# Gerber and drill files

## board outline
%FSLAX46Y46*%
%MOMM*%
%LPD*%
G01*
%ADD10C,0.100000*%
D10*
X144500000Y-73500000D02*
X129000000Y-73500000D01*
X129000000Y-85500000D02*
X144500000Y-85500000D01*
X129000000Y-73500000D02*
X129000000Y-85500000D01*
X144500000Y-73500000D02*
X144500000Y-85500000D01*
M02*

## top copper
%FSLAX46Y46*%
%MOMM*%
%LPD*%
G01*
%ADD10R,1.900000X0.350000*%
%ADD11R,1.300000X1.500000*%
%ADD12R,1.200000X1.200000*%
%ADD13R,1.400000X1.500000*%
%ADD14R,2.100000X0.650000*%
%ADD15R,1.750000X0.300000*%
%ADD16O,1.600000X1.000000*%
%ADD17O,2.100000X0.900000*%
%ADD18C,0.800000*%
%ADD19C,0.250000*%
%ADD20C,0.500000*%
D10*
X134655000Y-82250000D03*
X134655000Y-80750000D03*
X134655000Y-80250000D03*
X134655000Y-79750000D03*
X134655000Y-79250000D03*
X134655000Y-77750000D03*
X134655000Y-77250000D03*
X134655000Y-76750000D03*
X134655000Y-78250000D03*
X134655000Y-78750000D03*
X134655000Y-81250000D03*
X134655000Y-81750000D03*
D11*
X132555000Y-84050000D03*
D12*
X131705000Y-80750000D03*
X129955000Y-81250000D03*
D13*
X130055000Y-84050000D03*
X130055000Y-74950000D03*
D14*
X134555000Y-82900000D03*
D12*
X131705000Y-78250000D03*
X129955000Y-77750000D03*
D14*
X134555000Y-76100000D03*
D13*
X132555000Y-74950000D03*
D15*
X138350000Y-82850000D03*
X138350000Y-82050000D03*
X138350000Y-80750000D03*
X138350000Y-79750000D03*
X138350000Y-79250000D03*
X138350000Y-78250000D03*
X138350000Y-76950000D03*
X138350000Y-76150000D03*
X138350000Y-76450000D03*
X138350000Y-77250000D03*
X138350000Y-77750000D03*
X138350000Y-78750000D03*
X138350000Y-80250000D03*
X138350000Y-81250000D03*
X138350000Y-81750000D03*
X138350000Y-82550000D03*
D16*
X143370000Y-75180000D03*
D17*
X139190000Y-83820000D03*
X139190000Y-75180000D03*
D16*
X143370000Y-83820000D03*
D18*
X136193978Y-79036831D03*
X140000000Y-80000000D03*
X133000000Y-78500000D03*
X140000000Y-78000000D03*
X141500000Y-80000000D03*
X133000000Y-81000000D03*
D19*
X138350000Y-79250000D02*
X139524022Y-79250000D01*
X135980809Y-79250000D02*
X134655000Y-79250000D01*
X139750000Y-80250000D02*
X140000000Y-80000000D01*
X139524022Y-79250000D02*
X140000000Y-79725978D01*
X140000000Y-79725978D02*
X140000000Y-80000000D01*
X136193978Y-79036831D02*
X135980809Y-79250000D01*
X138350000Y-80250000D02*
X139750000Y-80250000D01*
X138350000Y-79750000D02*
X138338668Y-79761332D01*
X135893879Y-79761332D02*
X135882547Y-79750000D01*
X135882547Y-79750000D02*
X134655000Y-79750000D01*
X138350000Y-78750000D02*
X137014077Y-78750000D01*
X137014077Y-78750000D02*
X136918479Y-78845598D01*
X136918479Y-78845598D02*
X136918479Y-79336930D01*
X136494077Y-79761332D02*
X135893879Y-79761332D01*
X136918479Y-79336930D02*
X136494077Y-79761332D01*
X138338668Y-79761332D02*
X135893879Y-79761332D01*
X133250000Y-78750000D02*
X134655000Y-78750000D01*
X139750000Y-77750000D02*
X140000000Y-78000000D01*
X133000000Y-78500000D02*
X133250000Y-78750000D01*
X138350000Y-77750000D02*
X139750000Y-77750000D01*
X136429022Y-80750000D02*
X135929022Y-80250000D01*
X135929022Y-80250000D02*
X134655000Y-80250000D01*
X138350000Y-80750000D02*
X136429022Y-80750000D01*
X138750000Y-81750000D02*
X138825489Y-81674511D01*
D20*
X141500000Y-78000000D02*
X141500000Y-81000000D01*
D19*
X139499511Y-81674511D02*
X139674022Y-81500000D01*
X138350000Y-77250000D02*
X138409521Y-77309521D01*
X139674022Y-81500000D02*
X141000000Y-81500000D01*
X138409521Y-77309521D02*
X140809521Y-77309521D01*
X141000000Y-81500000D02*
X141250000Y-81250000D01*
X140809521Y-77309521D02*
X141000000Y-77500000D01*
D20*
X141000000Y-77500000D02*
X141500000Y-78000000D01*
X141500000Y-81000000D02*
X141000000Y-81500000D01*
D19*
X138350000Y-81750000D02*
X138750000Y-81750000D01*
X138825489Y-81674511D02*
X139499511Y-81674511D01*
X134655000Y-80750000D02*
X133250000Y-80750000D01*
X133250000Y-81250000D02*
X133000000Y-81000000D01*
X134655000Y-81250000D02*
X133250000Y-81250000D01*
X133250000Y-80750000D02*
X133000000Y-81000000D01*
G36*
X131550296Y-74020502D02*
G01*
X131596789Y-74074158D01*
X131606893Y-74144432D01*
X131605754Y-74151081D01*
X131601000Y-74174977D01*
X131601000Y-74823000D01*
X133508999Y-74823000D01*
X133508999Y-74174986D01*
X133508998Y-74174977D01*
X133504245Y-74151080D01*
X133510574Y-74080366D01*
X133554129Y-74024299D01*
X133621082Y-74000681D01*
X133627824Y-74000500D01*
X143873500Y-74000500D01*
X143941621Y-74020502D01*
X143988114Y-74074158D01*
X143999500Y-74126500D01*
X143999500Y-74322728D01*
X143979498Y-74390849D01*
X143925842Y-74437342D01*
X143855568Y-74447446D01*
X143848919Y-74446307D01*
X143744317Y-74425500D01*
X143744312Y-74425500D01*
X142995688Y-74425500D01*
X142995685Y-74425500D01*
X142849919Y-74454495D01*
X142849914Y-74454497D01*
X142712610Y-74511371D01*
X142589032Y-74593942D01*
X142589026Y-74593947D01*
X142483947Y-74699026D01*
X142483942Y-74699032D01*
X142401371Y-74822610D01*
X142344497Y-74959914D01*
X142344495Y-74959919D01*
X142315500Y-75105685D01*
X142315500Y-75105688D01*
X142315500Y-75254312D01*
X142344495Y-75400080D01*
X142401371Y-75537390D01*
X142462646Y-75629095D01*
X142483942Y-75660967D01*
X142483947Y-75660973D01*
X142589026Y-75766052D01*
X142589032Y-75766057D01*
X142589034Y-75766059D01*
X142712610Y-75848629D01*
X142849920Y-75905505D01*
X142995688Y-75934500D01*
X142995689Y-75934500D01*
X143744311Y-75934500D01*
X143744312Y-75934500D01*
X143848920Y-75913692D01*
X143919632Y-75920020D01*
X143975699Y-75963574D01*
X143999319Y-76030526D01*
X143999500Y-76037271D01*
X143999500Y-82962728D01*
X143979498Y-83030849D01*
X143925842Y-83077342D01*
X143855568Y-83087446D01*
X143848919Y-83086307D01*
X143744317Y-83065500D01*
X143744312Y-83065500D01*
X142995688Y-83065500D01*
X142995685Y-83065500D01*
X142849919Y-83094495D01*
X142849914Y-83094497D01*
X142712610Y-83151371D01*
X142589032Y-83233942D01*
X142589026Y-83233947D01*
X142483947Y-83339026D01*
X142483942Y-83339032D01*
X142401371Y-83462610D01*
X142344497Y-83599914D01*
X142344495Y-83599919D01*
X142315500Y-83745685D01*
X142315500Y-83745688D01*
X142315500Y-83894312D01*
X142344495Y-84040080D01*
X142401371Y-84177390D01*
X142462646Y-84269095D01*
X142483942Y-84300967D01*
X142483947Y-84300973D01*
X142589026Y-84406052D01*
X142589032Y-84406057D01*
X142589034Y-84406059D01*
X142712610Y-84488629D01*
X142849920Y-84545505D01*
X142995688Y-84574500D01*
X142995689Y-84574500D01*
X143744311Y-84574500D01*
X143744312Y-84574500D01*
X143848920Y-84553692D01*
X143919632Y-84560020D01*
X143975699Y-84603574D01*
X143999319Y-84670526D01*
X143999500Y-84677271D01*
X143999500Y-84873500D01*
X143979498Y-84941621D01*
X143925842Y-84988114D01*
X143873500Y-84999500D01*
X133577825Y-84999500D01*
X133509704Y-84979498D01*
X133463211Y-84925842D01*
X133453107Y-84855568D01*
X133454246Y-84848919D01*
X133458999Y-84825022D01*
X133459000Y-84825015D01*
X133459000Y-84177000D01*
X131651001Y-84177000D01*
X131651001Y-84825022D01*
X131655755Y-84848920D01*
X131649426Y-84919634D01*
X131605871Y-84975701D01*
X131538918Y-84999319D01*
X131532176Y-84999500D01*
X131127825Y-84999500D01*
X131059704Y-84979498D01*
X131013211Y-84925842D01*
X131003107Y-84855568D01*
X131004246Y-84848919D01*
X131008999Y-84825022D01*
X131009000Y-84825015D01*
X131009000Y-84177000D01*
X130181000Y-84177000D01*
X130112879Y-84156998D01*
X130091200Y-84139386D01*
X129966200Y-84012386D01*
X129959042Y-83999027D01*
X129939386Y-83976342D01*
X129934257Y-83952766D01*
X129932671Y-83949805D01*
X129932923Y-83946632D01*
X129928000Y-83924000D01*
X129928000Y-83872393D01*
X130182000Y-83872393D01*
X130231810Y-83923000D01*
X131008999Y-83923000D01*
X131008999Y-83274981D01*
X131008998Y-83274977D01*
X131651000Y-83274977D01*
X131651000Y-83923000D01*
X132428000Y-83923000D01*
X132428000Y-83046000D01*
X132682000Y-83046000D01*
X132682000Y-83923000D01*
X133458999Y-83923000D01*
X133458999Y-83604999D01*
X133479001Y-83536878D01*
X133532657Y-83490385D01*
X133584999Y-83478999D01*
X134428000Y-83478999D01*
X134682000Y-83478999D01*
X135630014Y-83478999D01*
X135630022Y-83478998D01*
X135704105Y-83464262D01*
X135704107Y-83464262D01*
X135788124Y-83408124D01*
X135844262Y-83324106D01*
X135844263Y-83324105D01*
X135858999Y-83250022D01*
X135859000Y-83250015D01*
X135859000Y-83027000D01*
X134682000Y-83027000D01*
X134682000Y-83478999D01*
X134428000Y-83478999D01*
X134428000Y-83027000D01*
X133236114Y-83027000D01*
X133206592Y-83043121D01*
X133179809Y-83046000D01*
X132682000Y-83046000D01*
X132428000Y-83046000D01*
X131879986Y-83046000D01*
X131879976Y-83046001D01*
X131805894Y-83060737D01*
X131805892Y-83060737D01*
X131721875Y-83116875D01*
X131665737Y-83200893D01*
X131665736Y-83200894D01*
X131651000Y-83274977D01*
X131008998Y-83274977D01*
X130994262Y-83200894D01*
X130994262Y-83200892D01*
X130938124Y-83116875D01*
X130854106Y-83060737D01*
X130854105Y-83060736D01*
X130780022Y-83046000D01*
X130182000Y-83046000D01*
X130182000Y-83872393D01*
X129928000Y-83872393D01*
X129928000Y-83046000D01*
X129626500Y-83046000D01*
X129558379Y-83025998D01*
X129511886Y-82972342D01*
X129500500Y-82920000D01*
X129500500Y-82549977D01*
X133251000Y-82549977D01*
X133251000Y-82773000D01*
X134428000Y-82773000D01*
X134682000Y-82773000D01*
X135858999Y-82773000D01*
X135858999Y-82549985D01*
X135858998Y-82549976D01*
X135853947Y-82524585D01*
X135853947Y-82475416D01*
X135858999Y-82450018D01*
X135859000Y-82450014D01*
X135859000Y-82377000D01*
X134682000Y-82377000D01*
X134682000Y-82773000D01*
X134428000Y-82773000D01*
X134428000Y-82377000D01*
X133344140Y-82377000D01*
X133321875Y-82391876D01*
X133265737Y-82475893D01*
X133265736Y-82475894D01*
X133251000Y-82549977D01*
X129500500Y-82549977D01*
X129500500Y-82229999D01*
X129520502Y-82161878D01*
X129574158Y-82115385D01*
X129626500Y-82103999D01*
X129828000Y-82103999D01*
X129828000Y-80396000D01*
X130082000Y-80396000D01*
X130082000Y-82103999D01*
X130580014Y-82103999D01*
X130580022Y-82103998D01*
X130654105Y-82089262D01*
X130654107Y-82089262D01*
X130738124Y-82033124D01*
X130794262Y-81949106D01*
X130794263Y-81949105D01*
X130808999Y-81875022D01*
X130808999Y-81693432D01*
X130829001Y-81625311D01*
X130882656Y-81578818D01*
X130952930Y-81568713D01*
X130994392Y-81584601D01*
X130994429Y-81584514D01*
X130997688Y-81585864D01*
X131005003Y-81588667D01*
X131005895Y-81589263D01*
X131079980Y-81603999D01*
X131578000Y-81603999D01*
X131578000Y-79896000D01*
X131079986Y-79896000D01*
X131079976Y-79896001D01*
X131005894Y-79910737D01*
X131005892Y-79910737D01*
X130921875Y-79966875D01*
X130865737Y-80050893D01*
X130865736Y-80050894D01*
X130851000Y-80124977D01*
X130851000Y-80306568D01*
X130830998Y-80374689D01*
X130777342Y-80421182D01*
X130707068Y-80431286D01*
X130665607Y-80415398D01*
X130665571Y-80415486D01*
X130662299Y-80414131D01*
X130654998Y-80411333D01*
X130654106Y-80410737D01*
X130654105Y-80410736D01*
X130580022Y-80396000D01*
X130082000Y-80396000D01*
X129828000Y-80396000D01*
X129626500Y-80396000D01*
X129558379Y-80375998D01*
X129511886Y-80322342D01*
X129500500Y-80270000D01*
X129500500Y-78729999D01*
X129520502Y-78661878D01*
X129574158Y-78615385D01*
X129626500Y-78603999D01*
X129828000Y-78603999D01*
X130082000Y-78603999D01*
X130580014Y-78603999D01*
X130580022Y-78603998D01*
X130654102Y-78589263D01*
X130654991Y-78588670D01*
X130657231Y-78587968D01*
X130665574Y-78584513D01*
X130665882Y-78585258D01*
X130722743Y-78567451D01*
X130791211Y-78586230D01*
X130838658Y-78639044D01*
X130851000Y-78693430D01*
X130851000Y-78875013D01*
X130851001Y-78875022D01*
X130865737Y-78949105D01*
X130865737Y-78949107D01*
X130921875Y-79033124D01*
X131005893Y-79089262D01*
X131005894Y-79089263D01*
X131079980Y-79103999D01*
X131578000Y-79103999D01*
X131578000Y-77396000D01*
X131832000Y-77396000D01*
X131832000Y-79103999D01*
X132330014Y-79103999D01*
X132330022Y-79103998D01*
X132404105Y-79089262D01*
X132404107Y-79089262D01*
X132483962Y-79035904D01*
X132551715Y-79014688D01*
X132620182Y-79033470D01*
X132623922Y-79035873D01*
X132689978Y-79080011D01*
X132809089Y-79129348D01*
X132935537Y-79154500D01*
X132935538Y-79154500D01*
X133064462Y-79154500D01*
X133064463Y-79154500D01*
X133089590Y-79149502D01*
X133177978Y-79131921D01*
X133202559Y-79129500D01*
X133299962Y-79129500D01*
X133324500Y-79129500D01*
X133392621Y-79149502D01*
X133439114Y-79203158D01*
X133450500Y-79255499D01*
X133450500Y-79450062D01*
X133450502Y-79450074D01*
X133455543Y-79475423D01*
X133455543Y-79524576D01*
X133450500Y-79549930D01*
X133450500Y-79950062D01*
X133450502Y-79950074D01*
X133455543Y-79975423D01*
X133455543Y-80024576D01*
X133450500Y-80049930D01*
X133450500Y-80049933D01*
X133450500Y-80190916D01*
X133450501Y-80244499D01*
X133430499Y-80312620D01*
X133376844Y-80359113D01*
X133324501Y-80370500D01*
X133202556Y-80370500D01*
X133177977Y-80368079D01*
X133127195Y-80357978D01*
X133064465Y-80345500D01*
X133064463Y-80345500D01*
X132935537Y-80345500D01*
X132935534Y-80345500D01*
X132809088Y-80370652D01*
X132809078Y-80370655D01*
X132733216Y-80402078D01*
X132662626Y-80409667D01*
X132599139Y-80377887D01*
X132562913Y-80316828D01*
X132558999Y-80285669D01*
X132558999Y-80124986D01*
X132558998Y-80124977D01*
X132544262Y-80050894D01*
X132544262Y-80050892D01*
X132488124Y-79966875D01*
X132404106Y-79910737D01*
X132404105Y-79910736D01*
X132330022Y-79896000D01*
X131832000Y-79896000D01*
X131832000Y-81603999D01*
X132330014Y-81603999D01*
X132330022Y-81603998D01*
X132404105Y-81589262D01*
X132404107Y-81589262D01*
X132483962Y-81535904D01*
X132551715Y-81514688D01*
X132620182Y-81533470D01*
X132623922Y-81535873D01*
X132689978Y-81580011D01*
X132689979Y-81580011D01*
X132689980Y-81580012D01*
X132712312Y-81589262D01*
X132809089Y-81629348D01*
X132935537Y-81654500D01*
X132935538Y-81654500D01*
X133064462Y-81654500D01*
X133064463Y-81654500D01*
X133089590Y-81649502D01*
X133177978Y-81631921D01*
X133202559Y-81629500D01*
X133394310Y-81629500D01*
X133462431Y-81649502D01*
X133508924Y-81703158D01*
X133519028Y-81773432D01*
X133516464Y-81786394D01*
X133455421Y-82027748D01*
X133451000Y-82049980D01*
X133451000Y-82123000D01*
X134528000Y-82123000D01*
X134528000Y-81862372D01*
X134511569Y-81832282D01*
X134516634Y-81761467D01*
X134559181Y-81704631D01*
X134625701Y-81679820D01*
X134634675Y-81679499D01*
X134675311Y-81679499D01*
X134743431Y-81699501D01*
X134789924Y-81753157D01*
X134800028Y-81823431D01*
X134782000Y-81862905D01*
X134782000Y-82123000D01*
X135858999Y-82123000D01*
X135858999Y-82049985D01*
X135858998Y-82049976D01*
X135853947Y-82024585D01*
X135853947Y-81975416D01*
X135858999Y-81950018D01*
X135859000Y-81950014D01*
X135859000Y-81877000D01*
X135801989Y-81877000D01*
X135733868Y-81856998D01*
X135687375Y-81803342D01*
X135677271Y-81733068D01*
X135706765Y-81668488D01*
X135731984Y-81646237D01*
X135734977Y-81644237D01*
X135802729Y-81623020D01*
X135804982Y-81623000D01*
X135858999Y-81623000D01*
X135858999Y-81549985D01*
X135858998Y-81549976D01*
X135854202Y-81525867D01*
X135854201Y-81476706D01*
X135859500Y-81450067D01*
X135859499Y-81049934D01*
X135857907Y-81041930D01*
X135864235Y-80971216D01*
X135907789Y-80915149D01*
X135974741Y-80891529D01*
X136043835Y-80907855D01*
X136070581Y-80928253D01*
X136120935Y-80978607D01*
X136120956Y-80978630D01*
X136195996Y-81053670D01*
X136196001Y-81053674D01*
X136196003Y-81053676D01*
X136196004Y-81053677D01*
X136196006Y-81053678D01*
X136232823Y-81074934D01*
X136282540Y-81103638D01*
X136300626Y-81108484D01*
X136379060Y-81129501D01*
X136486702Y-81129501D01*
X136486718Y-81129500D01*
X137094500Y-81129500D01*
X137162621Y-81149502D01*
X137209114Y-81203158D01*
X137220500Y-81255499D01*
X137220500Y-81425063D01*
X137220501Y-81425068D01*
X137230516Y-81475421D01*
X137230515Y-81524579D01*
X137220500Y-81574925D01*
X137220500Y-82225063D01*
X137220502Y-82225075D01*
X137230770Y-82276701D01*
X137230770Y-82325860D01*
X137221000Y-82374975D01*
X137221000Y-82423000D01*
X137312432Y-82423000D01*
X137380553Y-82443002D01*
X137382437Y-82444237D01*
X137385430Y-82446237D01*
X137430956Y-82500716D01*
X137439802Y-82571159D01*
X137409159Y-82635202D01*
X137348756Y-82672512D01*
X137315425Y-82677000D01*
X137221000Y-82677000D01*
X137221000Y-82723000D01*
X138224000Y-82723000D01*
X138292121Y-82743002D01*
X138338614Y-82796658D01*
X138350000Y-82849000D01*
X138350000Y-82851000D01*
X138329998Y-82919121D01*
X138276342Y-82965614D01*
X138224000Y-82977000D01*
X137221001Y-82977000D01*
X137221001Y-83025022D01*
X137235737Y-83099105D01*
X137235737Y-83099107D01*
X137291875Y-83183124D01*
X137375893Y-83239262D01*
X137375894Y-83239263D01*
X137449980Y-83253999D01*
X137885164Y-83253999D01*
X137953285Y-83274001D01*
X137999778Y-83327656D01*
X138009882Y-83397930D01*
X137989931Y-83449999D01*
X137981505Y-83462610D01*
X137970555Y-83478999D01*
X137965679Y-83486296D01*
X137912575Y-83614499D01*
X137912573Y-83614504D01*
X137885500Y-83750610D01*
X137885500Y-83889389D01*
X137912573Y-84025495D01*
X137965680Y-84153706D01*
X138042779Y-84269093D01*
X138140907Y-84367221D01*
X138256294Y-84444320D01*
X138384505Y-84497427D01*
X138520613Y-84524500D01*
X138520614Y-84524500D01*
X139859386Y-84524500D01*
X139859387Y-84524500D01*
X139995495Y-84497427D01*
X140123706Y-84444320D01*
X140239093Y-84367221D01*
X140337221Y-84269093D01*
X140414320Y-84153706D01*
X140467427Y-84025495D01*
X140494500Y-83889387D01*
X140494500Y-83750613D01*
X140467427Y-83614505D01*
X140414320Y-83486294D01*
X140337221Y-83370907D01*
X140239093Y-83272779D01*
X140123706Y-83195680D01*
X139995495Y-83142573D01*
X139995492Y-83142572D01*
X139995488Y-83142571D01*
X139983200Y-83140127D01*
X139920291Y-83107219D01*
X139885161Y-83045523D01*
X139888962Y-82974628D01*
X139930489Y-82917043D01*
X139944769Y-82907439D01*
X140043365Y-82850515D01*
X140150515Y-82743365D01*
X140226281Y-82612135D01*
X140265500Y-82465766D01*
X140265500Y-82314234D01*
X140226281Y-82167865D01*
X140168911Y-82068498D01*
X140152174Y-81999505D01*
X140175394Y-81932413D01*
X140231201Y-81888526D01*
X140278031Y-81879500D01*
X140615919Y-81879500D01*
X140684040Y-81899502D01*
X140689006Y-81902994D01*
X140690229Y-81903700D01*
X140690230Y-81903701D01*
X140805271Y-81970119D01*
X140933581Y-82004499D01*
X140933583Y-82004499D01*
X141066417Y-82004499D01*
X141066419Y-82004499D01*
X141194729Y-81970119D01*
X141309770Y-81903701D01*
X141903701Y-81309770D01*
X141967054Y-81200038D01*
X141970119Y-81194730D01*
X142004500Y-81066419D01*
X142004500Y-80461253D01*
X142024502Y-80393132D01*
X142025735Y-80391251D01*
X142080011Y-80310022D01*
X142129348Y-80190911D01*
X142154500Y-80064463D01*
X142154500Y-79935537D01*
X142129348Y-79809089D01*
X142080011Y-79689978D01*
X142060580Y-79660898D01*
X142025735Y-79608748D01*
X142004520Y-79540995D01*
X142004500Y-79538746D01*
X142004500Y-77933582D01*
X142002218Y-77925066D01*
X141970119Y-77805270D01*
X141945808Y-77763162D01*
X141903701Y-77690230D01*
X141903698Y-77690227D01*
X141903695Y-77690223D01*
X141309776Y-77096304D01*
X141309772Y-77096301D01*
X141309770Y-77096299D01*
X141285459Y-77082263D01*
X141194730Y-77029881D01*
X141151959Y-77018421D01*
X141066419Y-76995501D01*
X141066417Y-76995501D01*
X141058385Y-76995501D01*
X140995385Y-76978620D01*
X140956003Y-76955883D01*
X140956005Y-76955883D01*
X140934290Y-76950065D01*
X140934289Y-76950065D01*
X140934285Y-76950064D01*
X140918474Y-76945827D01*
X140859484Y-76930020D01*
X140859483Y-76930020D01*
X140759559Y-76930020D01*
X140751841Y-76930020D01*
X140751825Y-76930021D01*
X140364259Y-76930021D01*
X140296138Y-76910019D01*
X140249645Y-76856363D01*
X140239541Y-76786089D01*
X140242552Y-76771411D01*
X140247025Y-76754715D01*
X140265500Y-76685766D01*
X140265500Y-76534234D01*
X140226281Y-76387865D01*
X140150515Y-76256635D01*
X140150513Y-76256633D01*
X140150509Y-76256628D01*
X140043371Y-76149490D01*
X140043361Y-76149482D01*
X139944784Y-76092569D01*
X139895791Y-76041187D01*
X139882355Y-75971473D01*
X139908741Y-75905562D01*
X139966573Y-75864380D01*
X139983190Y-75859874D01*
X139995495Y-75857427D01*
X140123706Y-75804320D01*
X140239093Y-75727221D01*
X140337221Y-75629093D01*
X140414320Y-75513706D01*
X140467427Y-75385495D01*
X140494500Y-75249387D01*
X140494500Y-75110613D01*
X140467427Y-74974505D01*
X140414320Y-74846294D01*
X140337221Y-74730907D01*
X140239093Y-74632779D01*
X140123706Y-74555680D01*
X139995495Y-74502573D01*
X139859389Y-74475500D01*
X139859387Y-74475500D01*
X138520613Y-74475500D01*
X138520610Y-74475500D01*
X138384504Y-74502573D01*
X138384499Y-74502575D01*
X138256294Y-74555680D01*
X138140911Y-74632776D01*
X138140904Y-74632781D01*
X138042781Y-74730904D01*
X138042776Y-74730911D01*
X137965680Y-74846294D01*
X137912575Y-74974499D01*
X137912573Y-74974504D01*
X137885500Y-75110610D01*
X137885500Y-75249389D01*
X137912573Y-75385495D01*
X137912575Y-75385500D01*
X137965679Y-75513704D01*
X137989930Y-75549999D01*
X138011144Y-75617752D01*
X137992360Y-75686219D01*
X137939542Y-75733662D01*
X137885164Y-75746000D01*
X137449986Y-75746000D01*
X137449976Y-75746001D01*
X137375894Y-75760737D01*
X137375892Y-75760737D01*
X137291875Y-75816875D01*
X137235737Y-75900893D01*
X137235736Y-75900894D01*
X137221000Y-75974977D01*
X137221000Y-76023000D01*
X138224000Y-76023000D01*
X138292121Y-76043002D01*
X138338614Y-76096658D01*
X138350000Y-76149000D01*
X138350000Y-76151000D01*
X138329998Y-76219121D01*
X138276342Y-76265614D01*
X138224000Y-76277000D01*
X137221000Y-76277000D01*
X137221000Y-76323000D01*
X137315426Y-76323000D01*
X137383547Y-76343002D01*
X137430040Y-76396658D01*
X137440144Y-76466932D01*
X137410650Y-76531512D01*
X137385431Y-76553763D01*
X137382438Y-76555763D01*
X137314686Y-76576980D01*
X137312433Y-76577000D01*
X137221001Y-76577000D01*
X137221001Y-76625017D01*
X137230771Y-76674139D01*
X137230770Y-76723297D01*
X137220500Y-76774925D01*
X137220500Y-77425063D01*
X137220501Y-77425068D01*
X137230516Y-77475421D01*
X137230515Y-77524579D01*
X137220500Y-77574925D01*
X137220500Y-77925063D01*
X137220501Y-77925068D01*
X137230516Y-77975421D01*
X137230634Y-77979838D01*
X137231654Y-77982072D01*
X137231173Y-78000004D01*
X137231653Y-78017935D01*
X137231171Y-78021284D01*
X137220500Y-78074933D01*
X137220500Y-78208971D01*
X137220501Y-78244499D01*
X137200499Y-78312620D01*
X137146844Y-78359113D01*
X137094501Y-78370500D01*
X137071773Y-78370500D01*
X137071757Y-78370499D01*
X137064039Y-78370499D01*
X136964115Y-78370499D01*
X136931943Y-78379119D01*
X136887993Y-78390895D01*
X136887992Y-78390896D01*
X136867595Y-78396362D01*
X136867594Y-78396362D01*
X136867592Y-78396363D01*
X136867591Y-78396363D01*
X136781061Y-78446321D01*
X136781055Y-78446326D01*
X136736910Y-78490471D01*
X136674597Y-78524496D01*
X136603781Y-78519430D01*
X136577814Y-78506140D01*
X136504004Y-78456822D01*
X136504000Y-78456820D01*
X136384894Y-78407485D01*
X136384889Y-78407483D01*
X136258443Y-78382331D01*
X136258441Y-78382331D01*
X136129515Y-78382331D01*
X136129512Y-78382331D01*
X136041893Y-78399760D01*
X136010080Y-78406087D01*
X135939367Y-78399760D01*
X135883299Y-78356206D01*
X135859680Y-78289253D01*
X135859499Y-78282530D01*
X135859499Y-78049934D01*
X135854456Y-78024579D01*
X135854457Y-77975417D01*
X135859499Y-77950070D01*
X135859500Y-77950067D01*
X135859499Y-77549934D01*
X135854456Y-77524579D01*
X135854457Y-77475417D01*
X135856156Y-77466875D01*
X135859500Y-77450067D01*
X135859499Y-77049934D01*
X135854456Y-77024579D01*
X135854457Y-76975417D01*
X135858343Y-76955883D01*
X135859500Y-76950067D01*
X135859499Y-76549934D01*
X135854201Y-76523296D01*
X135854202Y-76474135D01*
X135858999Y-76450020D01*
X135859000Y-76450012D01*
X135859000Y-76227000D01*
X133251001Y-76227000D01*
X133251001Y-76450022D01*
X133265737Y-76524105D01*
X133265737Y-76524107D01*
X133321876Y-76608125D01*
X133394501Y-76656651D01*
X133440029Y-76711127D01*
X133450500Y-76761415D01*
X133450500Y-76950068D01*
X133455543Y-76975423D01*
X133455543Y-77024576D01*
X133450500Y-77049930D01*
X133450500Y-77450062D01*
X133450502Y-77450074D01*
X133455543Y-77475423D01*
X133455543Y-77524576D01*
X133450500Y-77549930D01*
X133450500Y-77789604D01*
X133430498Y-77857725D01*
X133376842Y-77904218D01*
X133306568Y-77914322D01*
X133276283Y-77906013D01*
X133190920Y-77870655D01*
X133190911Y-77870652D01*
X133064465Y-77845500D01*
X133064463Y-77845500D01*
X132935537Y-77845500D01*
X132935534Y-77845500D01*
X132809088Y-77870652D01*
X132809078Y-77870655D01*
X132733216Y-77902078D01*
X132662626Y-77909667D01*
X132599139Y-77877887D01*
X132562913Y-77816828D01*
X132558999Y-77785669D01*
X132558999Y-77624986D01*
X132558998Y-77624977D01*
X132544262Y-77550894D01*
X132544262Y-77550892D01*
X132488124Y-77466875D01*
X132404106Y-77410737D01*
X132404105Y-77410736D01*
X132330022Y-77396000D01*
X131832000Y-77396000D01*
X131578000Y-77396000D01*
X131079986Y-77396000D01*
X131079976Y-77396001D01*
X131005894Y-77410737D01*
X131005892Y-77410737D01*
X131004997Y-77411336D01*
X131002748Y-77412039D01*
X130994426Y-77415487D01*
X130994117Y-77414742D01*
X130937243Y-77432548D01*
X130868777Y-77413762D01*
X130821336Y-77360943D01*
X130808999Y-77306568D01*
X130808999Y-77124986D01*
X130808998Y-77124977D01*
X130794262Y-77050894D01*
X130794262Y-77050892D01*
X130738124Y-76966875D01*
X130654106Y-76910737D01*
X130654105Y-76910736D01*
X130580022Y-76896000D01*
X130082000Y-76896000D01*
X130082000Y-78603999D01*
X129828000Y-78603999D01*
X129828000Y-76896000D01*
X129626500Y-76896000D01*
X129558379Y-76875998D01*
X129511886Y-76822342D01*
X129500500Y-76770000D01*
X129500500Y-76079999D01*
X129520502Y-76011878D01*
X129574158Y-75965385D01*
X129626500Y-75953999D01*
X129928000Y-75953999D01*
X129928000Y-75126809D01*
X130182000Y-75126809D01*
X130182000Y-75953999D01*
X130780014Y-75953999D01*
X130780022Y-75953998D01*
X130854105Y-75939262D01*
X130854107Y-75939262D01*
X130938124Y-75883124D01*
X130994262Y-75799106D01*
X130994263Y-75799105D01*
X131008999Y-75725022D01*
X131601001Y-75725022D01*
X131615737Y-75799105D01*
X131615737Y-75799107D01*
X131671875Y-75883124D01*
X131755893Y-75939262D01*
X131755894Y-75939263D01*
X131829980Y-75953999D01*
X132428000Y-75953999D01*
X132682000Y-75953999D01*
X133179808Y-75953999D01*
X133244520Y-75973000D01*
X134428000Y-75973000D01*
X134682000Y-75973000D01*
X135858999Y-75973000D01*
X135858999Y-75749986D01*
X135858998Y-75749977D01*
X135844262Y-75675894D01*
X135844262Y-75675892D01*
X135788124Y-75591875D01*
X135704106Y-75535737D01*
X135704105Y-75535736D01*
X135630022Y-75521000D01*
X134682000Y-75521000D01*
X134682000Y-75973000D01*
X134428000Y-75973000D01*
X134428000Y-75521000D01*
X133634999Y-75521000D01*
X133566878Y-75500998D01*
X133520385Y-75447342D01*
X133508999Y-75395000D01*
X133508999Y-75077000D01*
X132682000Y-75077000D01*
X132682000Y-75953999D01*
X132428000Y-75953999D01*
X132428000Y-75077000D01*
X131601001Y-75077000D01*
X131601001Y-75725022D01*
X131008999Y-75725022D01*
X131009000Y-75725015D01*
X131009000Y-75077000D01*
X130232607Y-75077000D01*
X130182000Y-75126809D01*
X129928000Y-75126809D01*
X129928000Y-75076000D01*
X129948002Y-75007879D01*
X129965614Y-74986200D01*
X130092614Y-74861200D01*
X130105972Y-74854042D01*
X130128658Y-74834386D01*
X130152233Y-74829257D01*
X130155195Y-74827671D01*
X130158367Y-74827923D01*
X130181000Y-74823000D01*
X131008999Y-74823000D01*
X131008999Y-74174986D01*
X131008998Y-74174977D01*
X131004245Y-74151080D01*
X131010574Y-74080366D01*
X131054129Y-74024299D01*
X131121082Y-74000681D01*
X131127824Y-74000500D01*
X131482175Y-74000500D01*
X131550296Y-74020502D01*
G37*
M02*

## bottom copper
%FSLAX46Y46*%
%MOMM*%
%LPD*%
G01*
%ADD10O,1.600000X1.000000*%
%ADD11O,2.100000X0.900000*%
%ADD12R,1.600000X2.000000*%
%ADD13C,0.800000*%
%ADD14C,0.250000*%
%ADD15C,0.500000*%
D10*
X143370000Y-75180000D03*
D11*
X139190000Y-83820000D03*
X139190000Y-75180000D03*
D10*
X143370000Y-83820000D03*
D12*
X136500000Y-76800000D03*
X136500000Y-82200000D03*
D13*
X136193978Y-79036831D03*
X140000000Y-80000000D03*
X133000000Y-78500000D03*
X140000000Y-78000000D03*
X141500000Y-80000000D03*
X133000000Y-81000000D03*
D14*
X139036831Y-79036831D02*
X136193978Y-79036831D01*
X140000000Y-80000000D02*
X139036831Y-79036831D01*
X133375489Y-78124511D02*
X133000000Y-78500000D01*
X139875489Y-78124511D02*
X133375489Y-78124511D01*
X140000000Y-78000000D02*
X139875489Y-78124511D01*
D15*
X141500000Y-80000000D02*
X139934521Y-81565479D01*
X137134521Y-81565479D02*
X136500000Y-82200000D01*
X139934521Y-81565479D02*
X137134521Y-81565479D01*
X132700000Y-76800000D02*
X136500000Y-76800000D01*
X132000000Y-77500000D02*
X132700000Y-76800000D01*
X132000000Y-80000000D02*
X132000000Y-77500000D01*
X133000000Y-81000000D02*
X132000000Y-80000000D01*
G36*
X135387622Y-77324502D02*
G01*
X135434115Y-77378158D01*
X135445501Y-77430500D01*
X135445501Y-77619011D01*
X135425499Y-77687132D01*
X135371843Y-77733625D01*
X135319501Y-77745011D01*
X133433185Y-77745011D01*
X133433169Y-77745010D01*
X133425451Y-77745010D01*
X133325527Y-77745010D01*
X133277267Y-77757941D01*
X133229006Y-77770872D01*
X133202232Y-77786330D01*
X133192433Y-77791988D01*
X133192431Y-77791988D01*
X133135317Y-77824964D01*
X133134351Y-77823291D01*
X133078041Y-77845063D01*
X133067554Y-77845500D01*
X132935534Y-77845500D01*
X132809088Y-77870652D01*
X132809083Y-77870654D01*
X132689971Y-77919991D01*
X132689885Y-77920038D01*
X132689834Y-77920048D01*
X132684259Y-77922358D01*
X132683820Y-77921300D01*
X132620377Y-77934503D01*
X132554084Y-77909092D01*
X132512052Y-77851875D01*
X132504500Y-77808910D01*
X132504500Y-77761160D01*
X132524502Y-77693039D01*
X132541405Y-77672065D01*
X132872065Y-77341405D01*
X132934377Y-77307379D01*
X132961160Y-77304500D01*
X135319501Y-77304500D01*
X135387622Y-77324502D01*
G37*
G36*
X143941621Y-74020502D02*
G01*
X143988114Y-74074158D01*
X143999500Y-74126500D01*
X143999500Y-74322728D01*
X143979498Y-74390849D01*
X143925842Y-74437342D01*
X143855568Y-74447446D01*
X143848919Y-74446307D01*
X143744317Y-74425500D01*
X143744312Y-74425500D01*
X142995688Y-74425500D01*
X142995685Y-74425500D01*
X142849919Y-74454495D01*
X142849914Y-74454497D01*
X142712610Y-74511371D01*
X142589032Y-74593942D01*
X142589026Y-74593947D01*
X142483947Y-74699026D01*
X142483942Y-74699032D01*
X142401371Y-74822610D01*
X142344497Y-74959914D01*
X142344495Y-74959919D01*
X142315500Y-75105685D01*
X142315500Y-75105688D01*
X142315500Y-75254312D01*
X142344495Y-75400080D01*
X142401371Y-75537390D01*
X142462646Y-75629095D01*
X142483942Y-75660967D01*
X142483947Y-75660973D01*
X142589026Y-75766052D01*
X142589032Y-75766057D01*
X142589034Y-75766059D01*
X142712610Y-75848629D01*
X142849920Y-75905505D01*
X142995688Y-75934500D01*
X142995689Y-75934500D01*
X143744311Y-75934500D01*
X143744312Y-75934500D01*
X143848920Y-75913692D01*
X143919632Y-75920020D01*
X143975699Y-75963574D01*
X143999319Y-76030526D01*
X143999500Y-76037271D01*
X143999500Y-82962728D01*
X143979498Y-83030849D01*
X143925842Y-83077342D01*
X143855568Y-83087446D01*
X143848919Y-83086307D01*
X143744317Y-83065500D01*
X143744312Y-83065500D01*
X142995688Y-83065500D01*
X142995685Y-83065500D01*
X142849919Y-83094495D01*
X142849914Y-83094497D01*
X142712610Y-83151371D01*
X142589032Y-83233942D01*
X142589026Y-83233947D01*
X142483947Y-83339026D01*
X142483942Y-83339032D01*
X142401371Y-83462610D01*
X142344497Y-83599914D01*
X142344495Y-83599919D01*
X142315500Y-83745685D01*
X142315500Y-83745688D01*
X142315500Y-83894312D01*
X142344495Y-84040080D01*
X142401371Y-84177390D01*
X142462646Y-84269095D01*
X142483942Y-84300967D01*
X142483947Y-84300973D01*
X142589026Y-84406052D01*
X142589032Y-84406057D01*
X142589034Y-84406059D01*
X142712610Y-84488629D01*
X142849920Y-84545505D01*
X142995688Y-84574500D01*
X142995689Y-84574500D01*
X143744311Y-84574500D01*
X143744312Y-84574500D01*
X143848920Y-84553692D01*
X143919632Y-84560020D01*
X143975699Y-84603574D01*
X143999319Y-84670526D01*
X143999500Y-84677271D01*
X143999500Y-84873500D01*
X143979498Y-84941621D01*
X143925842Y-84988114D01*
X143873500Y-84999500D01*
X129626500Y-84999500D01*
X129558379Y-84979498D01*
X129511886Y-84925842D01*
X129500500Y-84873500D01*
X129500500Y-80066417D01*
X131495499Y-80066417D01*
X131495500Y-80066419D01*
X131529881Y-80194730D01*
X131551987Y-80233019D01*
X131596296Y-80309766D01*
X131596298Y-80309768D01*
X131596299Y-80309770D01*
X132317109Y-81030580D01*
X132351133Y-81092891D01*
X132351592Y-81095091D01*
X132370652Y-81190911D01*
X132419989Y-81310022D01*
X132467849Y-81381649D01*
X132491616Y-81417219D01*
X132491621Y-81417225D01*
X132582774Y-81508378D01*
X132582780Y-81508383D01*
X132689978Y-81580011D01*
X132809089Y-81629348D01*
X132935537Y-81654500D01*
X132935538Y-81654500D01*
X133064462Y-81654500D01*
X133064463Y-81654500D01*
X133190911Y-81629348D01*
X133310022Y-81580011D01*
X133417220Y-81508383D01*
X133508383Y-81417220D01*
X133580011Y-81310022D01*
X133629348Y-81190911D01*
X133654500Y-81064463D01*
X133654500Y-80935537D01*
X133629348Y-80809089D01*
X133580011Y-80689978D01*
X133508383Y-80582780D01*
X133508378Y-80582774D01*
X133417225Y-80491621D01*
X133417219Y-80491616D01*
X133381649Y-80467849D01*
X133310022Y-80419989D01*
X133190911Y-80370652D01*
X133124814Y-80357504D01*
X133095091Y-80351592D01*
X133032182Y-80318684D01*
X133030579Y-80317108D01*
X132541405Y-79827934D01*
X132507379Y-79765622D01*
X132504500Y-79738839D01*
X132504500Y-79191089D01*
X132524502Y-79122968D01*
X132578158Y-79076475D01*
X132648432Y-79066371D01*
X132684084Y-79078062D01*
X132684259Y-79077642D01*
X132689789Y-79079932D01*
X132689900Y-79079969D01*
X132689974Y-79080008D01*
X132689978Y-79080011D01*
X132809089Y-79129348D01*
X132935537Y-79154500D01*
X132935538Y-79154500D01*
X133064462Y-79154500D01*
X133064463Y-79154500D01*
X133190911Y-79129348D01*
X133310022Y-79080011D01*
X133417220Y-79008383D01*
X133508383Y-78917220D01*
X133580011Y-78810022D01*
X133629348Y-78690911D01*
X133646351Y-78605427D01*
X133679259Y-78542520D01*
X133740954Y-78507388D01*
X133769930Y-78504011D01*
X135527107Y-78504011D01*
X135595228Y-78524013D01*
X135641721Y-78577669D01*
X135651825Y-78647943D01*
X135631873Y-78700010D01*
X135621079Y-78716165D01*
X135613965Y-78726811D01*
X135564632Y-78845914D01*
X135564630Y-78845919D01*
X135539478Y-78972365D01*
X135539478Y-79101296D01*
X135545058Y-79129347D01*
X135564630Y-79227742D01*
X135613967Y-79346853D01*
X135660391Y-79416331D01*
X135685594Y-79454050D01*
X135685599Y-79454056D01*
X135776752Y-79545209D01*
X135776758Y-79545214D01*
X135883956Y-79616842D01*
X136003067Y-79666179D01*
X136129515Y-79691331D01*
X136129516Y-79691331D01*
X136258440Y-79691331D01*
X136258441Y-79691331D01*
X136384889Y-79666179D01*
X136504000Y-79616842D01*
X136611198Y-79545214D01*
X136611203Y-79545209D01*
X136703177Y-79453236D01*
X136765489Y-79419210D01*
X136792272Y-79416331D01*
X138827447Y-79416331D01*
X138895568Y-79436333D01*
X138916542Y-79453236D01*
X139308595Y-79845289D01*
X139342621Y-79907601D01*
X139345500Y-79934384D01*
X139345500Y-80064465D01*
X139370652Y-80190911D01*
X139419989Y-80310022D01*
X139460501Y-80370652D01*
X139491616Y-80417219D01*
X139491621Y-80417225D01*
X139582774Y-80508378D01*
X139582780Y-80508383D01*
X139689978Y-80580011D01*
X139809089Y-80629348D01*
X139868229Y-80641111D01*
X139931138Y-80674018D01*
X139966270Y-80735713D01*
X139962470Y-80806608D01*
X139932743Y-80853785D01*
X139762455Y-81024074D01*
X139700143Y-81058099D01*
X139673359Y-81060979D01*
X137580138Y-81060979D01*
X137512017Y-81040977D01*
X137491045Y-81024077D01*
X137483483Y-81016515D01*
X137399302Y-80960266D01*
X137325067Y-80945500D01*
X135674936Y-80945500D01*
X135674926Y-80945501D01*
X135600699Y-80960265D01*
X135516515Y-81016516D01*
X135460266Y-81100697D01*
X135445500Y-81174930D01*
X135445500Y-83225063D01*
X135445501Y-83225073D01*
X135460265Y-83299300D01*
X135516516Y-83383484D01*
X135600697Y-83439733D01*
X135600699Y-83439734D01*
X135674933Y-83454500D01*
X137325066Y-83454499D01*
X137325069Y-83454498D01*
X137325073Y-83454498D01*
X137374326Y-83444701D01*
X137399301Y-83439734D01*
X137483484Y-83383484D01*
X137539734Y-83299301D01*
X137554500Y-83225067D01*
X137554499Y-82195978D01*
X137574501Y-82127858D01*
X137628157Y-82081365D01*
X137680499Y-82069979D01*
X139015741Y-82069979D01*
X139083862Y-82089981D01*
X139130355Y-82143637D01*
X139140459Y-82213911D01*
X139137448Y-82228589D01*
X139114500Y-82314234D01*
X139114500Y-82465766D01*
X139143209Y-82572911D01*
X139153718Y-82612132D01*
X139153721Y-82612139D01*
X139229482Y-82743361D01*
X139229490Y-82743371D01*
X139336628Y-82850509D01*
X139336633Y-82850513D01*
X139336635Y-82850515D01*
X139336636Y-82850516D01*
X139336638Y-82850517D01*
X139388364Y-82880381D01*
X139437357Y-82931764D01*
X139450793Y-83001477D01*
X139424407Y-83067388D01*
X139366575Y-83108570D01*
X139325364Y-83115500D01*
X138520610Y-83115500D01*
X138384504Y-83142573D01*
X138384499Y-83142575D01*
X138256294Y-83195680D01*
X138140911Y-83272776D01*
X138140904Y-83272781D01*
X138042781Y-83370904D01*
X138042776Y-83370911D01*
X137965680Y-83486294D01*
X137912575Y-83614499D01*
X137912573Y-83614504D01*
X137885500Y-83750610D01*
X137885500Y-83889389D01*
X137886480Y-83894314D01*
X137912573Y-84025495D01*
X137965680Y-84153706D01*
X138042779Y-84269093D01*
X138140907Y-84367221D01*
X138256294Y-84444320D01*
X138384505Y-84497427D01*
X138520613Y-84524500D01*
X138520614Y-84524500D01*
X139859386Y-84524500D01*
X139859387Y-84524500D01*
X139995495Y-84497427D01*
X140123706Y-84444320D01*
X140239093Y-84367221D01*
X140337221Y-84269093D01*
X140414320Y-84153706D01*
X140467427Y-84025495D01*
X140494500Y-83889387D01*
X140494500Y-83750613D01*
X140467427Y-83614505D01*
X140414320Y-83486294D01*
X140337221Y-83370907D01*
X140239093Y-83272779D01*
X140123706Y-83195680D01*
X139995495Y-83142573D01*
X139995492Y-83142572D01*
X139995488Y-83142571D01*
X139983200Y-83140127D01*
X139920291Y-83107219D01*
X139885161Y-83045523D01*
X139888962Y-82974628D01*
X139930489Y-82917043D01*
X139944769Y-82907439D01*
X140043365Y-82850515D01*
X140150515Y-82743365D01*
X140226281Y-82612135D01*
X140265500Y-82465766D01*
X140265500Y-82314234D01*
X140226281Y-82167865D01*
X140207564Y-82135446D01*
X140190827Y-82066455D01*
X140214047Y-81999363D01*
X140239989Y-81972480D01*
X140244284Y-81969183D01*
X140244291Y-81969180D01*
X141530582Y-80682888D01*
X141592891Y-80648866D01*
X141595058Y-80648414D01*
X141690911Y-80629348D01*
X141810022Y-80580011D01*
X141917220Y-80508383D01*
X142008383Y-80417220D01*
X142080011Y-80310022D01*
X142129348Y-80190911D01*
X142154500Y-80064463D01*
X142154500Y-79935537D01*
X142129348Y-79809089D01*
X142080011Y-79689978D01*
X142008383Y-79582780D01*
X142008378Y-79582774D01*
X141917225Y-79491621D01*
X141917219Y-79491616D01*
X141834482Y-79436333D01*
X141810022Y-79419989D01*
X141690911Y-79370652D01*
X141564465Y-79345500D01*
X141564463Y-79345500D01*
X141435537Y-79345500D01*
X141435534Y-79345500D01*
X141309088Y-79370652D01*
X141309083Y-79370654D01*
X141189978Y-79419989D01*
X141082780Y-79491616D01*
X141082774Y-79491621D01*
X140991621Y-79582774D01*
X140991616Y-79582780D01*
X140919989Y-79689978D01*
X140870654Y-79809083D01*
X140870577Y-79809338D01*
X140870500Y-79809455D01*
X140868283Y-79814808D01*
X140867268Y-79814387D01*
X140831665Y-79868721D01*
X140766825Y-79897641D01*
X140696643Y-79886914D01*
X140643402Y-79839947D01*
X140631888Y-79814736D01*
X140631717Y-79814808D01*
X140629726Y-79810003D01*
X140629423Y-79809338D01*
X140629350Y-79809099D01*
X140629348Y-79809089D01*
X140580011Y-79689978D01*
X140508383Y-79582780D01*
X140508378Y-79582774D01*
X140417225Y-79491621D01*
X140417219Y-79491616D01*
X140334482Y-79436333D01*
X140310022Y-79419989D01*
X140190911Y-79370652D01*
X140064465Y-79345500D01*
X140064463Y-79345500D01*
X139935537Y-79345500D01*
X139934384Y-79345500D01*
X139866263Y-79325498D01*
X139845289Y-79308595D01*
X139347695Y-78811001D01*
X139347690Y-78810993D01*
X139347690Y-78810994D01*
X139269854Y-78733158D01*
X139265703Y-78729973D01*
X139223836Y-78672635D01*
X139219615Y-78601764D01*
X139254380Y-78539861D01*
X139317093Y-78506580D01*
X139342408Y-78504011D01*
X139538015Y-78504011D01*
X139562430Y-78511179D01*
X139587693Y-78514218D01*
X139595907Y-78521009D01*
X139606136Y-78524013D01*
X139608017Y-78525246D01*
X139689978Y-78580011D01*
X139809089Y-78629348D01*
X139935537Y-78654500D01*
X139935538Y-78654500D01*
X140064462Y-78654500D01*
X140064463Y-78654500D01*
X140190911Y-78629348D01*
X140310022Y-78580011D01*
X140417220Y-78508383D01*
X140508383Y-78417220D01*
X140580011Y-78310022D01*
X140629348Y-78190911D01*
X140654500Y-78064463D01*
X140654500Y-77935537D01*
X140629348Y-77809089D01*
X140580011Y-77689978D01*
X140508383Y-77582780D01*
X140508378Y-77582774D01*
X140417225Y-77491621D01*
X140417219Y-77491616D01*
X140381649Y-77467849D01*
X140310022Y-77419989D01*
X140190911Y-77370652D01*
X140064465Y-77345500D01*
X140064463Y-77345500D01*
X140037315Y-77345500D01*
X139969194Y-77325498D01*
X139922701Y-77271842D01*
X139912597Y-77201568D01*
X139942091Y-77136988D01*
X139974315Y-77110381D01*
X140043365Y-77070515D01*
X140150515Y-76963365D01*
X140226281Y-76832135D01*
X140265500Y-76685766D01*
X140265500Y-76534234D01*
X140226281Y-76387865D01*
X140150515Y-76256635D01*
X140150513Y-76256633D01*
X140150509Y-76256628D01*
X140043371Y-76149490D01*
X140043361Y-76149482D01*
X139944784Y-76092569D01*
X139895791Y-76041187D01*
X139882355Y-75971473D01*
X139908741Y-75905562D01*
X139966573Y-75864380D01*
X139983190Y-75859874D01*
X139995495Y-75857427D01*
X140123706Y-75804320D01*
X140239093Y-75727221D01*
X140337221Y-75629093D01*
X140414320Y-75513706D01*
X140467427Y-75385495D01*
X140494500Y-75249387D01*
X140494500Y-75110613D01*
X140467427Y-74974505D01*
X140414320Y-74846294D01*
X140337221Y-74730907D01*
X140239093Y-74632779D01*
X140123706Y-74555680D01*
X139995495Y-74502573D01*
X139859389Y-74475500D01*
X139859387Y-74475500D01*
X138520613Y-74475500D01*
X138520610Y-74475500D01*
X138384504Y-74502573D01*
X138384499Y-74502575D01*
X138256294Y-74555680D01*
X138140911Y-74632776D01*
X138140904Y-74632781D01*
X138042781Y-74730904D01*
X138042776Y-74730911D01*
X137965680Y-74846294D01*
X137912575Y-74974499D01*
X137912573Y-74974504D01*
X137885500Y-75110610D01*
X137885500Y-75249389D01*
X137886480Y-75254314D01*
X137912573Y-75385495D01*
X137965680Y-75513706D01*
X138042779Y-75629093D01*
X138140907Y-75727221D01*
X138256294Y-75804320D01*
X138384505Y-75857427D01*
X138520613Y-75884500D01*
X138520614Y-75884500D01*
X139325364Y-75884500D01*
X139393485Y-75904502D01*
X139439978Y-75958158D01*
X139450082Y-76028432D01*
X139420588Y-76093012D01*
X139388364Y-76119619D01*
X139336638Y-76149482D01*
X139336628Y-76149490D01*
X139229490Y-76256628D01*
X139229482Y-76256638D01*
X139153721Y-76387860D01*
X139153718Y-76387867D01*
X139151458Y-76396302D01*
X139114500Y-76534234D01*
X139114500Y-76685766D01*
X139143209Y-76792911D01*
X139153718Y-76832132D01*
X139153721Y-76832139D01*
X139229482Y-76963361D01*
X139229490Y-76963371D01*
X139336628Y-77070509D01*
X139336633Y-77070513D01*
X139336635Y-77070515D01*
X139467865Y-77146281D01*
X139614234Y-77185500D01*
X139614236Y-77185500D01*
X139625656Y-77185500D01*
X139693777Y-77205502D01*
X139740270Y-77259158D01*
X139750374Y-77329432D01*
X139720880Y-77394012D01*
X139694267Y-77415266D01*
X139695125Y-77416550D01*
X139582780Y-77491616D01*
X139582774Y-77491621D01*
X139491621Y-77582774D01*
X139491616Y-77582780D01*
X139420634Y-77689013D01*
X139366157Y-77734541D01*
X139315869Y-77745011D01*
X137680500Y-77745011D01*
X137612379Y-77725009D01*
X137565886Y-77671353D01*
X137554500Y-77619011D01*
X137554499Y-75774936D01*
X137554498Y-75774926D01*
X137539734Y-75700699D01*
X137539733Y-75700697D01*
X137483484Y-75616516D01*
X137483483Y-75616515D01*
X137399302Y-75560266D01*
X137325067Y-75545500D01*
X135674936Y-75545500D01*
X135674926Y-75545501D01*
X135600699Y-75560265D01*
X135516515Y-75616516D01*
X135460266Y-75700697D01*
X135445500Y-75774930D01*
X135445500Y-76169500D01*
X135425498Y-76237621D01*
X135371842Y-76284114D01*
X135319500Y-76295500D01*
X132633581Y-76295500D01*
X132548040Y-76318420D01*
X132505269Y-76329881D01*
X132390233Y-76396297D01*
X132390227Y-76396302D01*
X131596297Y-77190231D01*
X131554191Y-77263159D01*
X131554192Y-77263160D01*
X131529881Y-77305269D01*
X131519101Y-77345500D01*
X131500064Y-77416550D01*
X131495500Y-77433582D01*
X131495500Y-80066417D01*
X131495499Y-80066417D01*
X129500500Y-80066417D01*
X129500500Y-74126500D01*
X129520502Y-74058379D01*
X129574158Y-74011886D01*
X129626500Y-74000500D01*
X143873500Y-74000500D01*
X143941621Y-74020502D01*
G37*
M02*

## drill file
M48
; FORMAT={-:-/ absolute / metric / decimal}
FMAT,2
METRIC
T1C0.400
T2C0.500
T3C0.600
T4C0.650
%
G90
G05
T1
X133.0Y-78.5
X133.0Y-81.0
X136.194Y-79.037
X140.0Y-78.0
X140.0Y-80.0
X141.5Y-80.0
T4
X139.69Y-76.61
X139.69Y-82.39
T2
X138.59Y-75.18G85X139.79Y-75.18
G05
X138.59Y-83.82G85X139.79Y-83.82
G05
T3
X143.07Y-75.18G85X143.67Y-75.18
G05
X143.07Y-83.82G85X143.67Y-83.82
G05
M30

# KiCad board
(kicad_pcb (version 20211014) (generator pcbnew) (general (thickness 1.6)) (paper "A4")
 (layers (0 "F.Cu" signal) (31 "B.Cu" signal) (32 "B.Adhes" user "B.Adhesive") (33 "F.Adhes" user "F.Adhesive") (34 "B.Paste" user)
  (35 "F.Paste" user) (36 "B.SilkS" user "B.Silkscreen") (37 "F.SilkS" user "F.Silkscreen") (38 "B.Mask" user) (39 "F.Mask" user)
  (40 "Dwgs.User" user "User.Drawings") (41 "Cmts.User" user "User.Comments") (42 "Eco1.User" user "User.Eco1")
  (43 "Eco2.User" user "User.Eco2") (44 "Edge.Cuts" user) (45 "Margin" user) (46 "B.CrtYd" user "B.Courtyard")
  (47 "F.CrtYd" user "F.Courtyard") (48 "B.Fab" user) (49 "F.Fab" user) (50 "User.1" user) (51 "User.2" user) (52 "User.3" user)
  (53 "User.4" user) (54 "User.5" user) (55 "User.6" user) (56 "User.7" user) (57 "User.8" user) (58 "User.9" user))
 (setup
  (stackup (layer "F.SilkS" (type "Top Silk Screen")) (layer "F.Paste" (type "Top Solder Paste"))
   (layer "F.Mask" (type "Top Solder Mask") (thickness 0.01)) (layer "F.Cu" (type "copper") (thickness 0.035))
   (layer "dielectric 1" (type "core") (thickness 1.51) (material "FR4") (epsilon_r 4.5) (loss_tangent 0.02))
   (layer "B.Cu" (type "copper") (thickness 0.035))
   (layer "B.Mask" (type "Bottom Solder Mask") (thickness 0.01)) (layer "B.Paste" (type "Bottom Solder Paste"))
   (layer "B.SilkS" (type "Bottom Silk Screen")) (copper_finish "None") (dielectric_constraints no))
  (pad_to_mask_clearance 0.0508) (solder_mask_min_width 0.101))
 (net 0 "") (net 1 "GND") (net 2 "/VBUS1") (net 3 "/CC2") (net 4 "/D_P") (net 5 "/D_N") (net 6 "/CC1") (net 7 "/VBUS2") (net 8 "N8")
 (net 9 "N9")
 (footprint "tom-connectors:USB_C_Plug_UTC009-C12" (layer "F.Cu") (at 134.455 79.5 -90)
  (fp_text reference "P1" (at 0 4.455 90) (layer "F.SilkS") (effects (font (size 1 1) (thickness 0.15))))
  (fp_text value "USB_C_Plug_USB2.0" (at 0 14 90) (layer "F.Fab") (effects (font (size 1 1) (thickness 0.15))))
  (pad "A1" smd rect (at 2.75 -0.2 270) (size 0.35 1.9) (layers "F.Cu" "F.Paste" "F.Mask") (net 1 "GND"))
  (pad "A4" smd rect (at 1.25 -0.2 270) (size 0.35 1.9) (layers "F.Cu" "F.Paste" "F.Mask") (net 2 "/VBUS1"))
  (pad "A5" smd rect (at 0.75 -0.2 270) (size 0.35 1.9) (layers "F.Cu" "F.Paste" "F.Mask") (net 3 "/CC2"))
  (pad "A6" smd rect (at 0.25 -0.2 270) (size 0.35 1.9) (layers "F.Cu" "F.Paste" "F.Mask") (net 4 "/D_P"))
  (pad "A7" smd rect (at -0.25 -0.2 270) (size 0.35 1.9) (layers "F.Cu" "F.Paste" "F.Mask") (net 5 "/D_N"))
  (pad "A10" smd rect (at -1.75 -0.2 270) (size 0.35 1.9) (layers "F.Cu" "F.Paste" "F.Mask"))
  (pad "A11" smd rect (at -2.25 -0.2 270) (size 0.35 1.9) (layers "F.Cu" "F.Paste" "F.Mask"))
  (pad "B2" smd rect (at -2.75 -0.2 270) (size 0.35 1.9) (layers "F.Cu" "F.Paste" "F.Mask"))
  (pad "B3" smd rect (at -1.25 -0.2 270) (size 0.35 1.9) (layers "F.Cu" "F.Paste" "F.Mask"))
  (pad "B5" smd rect (at -0.75 -0.2 270) (size 0.35 1.9) (layers "F.Cu" "F.Paste" "F.Mask") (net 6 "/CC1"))
  (pad "B9" smd rect (at 1.75 -0.2 270) (size 0.35 1.9) (layers "F.Cu" "F.Paste" "F.Mask") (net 2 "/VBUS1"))
  (pad "B12" smd rect (at 2.25 -0.2 270) (size 0.35 1.9) (layers "F.Cu" "F.Paste" "F.Mask") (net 1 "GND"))
  (pad "S1" smd rect (at 4.55 1.9 270) (size 1.5 1.3) (layers "F.Cu" "F.Paste" "F.Mask") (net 1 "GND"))
  (pad "S1" smd rect (at 1.25 2.75 270) (size 1.2 1.2) (layers "F.Cu" "F.Paste" "F.Mask") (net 1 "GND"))
  (pad "S1" smd rect (at 1.75 4.5 270) (size 1.2 1.2) (layers "F.Cu" "F.Paste" "F.Mask") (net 1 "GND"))
  (pad "S1" smd rect (at 4.55 4.4 270) (size 1.5 1.4) (layers "F.Cu" "F.Paste" "F.Mask") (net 1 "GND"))
  (pad "S1" smd rect (at -4.55 4.4 270) (size 1.5 1.4) (layers "F.Cu" "F.Paste" "F.Mask") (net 1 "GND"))
  (pad "S1" smd rect (at 3.4 -0.1 270) (size 0.65 2.1) (layers "F.Cu" "F.Paste" "F.Mask") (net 1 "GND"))
  (pad "S1" smd rect (at -1.25 2.75 270) (size 1.2 1.2) (layers "F.Cu" "F.Paste" "F.Mask") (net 1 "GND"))
  (pad "S1" smd rect (at -1.75 4.5 270) (size 1.2 1.2) (layers "F.Cu" "F.Paste" "F.Mask") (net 1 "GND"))
  (pad "S1" smd rect (at -3.4 -0.1 270) (size 0.65 2.1) (layers "F.Cu" "F.Paste" "F.Mask") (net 1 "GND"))
  (pad "S1" smd rect (at -4.55 1.9 270) (size 1.5 1.4) (layers "F.Cu" "F.Paste" "F.Mask") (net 1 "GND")))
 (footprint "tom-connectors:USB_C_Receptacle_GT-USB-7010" (layer "F.Cu") (at 141.5 79.5 90)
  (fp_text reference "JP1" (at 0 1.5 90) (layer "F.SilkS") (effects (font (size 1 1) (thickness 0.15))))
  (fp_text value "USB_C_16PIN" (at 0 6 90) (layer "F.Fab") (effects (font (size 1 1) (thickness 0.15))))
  (pad "" np_thru_hole circle locked (at 2.89 -1.81 90) (size 0.65 0.65) (drill 0.65) (layers *.Cu *.Mask))
  (pad "" np_thru_hole circle locked (at -2.89 -1.81 90) (size 0.65 0.65) (drill 0.65) (layers *.Cu *.Mask))
  (pad "A1" smd rect locked (at -3.35 -3.15 90) (size 0.3 1.75) (layers "F.Cu" "F.Paste" "F.Mask") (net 1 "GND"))
  (pad "A4" smd rect locked (at -2.55 -3.15 90) (size 0.3 1.75) (layers "F.Cu" "F.Paste" "F.Mask") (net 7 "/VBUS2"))
  (pad "A5" smd rect locked (at -1.25 -3.15 90) (size 0.3 1.75) (layers "F.Cu" "F.Paste" "F.Mask") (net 3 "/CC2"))
  (pad "A6" smd rect locked (at -0.25 -3.15 90) (size 0.3 1.75) (layers "F.Cu" "F.Paste" "F.Mask") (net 4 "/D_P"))
  (pad "A7" smd rect locked (at 0.25 -3.15 90) (size 0.3 1.75) (layers "F.Cu" "F.Paste" "F.Mask") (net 5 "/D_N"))
  (pad "A8" smd rect locked (at 1.25 -3.15 90) (size 0.3 1.75) (layers "F.Cu" "F.Paste" "F.Mask") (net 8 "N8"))
  (pad "A9" smd rect locked (at 2.55 -3.15 90) (size 0.3 1.75) (layers "F.Cu" "F.Paste" "F.Mask") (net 7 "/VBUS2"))
  (pad "A12" smd rect locked (at 3.35 -3.15 90) (size 0.3 1.75) (layers "F.Cu" "F.Paste" "F.Mask") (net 1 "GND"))
  (pad "B1" smd rect locked (at 3.05 -3.15 90) (size 0.3 1.75) (layers "F.Cu" "F.Paste" "F.Mask") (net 1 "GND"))
  (pad "B4" smd rect locked (at 2.25 -3.15 90) (size 0.3 1.75) (layers "F.Cu" "F.Paste" "F.Mask") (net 7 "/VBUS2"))
  (pad "B5" smd rect locked (at 1.75 -3.15 90) (size 0.3 1.75) (layers "F.Cu" "F.Paste" "F.Mask") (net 6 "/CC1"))
  (pad "B6" smd rect locked (at 0.75 -3.15 90) (size 0.3 1.75) (layers "F.Cu" "F.Paste" "F.Mask") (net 4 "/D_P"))
  (pad "B7" smd rect locked (at -0.75 -3.15 90) (size 0.3 1.75) (layers "F.Cu" "F.Paste" "F.Mask") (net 5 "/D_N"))
  (pad "B8" smd rect locked (at -1.75 -3.15 90) (size 0.3 1.75) (layers "F.Cu" "F.Paste" "F.Mask") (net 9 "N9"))
  (pad "B9" smd rect locked (at -2.25 -3.15 90) (size 0.3 1.75) (layers "F.Cu" "F.Paste" "F.Mask") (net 7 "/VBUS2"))
  (pad "B12" smd rect locked (at -3.05 -3.15 90) (size 0.3 1.75) (layers "F.Cu" "F.Paste" "F.Mask") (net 1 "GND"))
  (pad "S1" thru_hole oval locked (at 4.32 1.87 90) (size 1 1.6) (drill oval 0.6 1.2) (layers *.Cu *.Paste *.Mask))
  (pad "S1" thru_hole oval locked (at -4.32 -2.31 90) (size 0.9 2.1) (drill oval 0.5 1.7) (layers *.Cu *.Paste *.Mask))
  (pad "S1" thru_hole oval locked (at 4.32 -2.31 90) (size 0.9 2.1) (drill oval 0.5 1.7) (layers *.Cu *.Paste *.Mask))
  (pad "S1" thru_hole oval locked (at -4.32 1.87 90) (size 1 1.6) (drill oval 0.6 1.2) (layers *.Cu *.Paste *.Mask)))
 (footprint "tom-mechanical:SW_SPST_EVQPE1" (layer "B.Cu") (at 136.5 79.5 -90)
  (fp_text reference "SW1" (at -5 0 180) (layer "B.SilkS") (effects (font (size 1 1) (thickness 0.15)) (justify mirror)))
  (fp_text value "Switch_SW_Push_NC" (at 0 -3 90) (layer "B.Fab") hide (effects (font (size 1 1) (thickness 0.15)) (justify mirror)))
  (pad "1" smd rect (at -2.7 0 270) (size 2 1.6) (layers "B.Cu" "B.Paste" "B.Mask") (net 2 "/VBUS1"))
  (pad "2" smd rect (at 2.7 0 270) (size 2 1.6) (layers "B.Cu" "B.Paste" "B.Mask") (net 7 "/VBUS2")))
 (gr_line (start 144.5 73.5) (end 129 73.5) (layer "Edge.Cuts") (width 0.1))
 (gr_line (start 129 85.5) (end 144.5 85.5) (layer "Edge.Cuts") (width 0.1))
 (gr_line (start 129 73.5) (end 129 85.5) (layer "Edge.Cuts") (width 0.1))
 (gr_line (start 144.5 73.5) (end 144.5 85.5) (layer "Edge.Cuts") (width 0.1))
 (segment (start 138.35 79.25) (end 139.524022 79.25) (width 0.25) (layer "F.Cu") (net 5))
 (segment (start 135.980809 79.25) (end 134.655 79.25) (width 0.25) (layer "F.Cu") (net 5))
 (segment (start 139.75 80.25) (end 140 80) (width 0.25) (layer "F.Cu") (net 5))
 (segment (start 139.524022 79.25) (end 140 79.725978) (width 0.25) (layer "F.Cu") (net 5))
 (segment (start 140 79.725978) (end 140 80) (width 0.25) (layer "F.Cu") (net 5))
 (segment (start 136.193978 79.036831) (end 135.980809 79.25) (width 0.25) (layer "F.Cu") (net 5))
 (segment (start 138.35 80.25) (end 139.75 80.25) (width 0.25) (layer "F.Cu") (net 5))
 (via (at 136.193978 79.036831) (size 0.8) (drill 0.4) (layers "F.Cu" "B.Cu") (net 5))
 (via (at 140 80) (size 0.8) (drill 0.4) (layers "F.Cu" "B.Cu") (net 5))
 (segment (start 139.036831 79.036831) (end 136.193978 79.036831) (width 0.25) (layer "B.Cu") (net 5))
 (segment (start 140 80) (end 139.036831 79.036831) (width 0.25) (layer "B.Cu") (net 5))
 (segment (start 138.35 79.75) (end 138.338668 79.761332) (width 0.25) (layer "F.Cu") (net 4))
 (segment (start 135.893879 79.761332) (end 135.882547 79.75) (width 0.25) (layer "F.Cu") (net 4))
 (segment (start 135.882547 79.75) (end 134.655 79.75) (width 0.25) (layer "F.Cu") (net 4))
 (segment (start 138.35 78.75) (end 137.014077 78.75) (width 0.25) (layer "F.Cu") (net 4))
 (segment (start 137.014077 78.75) (end 136.918479 78.845598) (width 0.25) (layer "F.Cu") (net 4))
 (segment (start 136.918479 78.845598) (end 136.918479 79.33693) (width 0.25) (layer "F.Cu") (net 4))
 (segment (start 136.494077 79.761332) (end 135.893879 79.761332) (width 0.25) (layer "F.Cu") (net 4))
 (segment (start 136.918479 79.33693) (end 136.494077 79.761332) (width 0.25) (layer "F.Cu") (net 4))
 (segment (start 138.338668 79.761332) (end 135.893879 79.761332) (width 0.25) (layer "F.Cu") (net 4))
 (segment (start 133.25 78.75) (end 134.655 78.75) (width 0.25) (layer "F.Cu") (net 6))
 (segment (start 139.75 77.75) (end 140 78) (width 0.25) (layer "F.Cu") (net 6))
 (segment (start 133 78.5) (end 133.25 78.75) (width 0.25) (layer "F.Cu") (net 6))
 (segment (start 138.35 77.75) (end 139.75 77.75) (width 0.25) (layer "F.Cu") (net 6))
 (via (at 133 78.5) (size 0.8) (drill 0.4) (layers "F.Cu" "B.Cu") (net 6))
 (via (at 140 78) (size 0.8) (drill 0.4) (layers "F.Cu" "B.Cu") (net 6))
 (segment (start 133.375489 78.124511) (end 133 78.5) (width 0.25) (layer "B.Cu") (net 6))
 (segment (start 139.875489 78.124511) (end 133.375489 78.124511) (width 0.25) (layer "B.Cu") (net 6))
 (segment (start 140 78) (end 139.875489 78.124511) (width 0.25) (layer "B.Cu") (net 6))
 (segment (start 136.429022 80.75) (end 135.929022 80.25) (width 0.25) (layer "F.Cu") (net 3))
 (segment (start 135.929022 80.25) (end 134.655 80.25) (width 0.25) (layer "F.Cu") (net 3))
 (segment (start 138.35 80.75) (end 136.429022 80.75) (width 0.25) (layer "F.Cu") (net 3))
 (segment (start 138.75 81.75) (end 138.825489 81.674511) (width 0.25) (layer "F.Cu") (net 7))
 (segment (start 141.5 78) (end 141.5 81) (width 0.5) (layer "F.Cu") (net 7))
 (segment (start 139.499511 81.674511) (end 139.674022 81.5) (width 0.25) (layer "F.Cu") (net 7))
 (segment (start 138.35 77.25) (end 138.409521 77.309521) (width 0.25) (layer "F.Cu") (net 7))
 (segment (start 139.674022 81.5) (end 141 81.5) (width 0.25) (layer "F.Cu") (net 7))
 (segment (start 138.409521 77.309521) (end 140.809521 77.309521) (width 0.25) (layer "F.Cu") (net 7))
 (segment (start 141 81.5) (end 141.25 81.25) (width 0.25) (layer "F.Cu") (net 7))
 (segment (start 140.809521 77.309521) (end 141 77.5) (width 0.25) (layer "F.Cu") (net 7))
 (segment (start 141 77.5) (end 141.5 78) (width 0.5) (layer "F.Cu") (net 7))
 (segment (start 141.5 81) (end 141 81.5) (width 0.5) (layer "F.Cu") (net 7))
 (segment (start 138.35 81.75) (end 138.75 81.75) (width 0.25) (layer "F.Cu") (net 7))
 (segment (start 138.825489 81.674511) (end 139.499511 81.674511) (width 0.25) (layer "F.Cu") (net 7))
 (via (at 141.5 80) (size 0.8) (drill 0.4) (layers "F.Cu" "B.Cu") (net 7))
 (segment (start 141.5 80) (end 139.934521 81.565479) (width 0.5) (layer "B.Cu") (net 7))
 (segment (start 137.134521 81.565479) (end 136.5 82.2) (width 0.5) (layer "B.Cu") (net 7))
 (segment (start 139.934521 81.565479) (end 137.134521 81.565479) (width 0.5) (layer "B.Cu") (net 7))
 (segment (start 134.655 80.75) (end 133.25 80.75) (width 0.25) (layer "F.Cu") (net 2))
 (segment (start 133.25 81.25) (end 133 81) (width 0.25) (layer "F.Cu") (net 2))
 (segment (start 134.655 81.25) (end 133.25 81.25) (width 0.25) (layer "F.Cu") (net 2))
 (segment (start 133.25 80.75) (end 133 81) (width 0.25) (layer "F.Cu") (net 2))
 (via (at 133 81) (size 0.8) (drill 0.4) (layers "F.Cu" "B.Cu") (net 2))
 (segment (start 132.7 76.8) (end 136.5 76.8) (width 0.5) (layer "B.Cu") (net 2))
 (segment (start 132 77.5) (end 132.7 76.8) (width 0.5) (layer "B.Cu") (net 2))
 (segment (start 132 80) (end 132 77.5) (width 0.5) (layer "B.Cu") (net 2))
 (segment (start 133 81) (end 132 80) (width 0.5) (layer "B.Cu") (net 2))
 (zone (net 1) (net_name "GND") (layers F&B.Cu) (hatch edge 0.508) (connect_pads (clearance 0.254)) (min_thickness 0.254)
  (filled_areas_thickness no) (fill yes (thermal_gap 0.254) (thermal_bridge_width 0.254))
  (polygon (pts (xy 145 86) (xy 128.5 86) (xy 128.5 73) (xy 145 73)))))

